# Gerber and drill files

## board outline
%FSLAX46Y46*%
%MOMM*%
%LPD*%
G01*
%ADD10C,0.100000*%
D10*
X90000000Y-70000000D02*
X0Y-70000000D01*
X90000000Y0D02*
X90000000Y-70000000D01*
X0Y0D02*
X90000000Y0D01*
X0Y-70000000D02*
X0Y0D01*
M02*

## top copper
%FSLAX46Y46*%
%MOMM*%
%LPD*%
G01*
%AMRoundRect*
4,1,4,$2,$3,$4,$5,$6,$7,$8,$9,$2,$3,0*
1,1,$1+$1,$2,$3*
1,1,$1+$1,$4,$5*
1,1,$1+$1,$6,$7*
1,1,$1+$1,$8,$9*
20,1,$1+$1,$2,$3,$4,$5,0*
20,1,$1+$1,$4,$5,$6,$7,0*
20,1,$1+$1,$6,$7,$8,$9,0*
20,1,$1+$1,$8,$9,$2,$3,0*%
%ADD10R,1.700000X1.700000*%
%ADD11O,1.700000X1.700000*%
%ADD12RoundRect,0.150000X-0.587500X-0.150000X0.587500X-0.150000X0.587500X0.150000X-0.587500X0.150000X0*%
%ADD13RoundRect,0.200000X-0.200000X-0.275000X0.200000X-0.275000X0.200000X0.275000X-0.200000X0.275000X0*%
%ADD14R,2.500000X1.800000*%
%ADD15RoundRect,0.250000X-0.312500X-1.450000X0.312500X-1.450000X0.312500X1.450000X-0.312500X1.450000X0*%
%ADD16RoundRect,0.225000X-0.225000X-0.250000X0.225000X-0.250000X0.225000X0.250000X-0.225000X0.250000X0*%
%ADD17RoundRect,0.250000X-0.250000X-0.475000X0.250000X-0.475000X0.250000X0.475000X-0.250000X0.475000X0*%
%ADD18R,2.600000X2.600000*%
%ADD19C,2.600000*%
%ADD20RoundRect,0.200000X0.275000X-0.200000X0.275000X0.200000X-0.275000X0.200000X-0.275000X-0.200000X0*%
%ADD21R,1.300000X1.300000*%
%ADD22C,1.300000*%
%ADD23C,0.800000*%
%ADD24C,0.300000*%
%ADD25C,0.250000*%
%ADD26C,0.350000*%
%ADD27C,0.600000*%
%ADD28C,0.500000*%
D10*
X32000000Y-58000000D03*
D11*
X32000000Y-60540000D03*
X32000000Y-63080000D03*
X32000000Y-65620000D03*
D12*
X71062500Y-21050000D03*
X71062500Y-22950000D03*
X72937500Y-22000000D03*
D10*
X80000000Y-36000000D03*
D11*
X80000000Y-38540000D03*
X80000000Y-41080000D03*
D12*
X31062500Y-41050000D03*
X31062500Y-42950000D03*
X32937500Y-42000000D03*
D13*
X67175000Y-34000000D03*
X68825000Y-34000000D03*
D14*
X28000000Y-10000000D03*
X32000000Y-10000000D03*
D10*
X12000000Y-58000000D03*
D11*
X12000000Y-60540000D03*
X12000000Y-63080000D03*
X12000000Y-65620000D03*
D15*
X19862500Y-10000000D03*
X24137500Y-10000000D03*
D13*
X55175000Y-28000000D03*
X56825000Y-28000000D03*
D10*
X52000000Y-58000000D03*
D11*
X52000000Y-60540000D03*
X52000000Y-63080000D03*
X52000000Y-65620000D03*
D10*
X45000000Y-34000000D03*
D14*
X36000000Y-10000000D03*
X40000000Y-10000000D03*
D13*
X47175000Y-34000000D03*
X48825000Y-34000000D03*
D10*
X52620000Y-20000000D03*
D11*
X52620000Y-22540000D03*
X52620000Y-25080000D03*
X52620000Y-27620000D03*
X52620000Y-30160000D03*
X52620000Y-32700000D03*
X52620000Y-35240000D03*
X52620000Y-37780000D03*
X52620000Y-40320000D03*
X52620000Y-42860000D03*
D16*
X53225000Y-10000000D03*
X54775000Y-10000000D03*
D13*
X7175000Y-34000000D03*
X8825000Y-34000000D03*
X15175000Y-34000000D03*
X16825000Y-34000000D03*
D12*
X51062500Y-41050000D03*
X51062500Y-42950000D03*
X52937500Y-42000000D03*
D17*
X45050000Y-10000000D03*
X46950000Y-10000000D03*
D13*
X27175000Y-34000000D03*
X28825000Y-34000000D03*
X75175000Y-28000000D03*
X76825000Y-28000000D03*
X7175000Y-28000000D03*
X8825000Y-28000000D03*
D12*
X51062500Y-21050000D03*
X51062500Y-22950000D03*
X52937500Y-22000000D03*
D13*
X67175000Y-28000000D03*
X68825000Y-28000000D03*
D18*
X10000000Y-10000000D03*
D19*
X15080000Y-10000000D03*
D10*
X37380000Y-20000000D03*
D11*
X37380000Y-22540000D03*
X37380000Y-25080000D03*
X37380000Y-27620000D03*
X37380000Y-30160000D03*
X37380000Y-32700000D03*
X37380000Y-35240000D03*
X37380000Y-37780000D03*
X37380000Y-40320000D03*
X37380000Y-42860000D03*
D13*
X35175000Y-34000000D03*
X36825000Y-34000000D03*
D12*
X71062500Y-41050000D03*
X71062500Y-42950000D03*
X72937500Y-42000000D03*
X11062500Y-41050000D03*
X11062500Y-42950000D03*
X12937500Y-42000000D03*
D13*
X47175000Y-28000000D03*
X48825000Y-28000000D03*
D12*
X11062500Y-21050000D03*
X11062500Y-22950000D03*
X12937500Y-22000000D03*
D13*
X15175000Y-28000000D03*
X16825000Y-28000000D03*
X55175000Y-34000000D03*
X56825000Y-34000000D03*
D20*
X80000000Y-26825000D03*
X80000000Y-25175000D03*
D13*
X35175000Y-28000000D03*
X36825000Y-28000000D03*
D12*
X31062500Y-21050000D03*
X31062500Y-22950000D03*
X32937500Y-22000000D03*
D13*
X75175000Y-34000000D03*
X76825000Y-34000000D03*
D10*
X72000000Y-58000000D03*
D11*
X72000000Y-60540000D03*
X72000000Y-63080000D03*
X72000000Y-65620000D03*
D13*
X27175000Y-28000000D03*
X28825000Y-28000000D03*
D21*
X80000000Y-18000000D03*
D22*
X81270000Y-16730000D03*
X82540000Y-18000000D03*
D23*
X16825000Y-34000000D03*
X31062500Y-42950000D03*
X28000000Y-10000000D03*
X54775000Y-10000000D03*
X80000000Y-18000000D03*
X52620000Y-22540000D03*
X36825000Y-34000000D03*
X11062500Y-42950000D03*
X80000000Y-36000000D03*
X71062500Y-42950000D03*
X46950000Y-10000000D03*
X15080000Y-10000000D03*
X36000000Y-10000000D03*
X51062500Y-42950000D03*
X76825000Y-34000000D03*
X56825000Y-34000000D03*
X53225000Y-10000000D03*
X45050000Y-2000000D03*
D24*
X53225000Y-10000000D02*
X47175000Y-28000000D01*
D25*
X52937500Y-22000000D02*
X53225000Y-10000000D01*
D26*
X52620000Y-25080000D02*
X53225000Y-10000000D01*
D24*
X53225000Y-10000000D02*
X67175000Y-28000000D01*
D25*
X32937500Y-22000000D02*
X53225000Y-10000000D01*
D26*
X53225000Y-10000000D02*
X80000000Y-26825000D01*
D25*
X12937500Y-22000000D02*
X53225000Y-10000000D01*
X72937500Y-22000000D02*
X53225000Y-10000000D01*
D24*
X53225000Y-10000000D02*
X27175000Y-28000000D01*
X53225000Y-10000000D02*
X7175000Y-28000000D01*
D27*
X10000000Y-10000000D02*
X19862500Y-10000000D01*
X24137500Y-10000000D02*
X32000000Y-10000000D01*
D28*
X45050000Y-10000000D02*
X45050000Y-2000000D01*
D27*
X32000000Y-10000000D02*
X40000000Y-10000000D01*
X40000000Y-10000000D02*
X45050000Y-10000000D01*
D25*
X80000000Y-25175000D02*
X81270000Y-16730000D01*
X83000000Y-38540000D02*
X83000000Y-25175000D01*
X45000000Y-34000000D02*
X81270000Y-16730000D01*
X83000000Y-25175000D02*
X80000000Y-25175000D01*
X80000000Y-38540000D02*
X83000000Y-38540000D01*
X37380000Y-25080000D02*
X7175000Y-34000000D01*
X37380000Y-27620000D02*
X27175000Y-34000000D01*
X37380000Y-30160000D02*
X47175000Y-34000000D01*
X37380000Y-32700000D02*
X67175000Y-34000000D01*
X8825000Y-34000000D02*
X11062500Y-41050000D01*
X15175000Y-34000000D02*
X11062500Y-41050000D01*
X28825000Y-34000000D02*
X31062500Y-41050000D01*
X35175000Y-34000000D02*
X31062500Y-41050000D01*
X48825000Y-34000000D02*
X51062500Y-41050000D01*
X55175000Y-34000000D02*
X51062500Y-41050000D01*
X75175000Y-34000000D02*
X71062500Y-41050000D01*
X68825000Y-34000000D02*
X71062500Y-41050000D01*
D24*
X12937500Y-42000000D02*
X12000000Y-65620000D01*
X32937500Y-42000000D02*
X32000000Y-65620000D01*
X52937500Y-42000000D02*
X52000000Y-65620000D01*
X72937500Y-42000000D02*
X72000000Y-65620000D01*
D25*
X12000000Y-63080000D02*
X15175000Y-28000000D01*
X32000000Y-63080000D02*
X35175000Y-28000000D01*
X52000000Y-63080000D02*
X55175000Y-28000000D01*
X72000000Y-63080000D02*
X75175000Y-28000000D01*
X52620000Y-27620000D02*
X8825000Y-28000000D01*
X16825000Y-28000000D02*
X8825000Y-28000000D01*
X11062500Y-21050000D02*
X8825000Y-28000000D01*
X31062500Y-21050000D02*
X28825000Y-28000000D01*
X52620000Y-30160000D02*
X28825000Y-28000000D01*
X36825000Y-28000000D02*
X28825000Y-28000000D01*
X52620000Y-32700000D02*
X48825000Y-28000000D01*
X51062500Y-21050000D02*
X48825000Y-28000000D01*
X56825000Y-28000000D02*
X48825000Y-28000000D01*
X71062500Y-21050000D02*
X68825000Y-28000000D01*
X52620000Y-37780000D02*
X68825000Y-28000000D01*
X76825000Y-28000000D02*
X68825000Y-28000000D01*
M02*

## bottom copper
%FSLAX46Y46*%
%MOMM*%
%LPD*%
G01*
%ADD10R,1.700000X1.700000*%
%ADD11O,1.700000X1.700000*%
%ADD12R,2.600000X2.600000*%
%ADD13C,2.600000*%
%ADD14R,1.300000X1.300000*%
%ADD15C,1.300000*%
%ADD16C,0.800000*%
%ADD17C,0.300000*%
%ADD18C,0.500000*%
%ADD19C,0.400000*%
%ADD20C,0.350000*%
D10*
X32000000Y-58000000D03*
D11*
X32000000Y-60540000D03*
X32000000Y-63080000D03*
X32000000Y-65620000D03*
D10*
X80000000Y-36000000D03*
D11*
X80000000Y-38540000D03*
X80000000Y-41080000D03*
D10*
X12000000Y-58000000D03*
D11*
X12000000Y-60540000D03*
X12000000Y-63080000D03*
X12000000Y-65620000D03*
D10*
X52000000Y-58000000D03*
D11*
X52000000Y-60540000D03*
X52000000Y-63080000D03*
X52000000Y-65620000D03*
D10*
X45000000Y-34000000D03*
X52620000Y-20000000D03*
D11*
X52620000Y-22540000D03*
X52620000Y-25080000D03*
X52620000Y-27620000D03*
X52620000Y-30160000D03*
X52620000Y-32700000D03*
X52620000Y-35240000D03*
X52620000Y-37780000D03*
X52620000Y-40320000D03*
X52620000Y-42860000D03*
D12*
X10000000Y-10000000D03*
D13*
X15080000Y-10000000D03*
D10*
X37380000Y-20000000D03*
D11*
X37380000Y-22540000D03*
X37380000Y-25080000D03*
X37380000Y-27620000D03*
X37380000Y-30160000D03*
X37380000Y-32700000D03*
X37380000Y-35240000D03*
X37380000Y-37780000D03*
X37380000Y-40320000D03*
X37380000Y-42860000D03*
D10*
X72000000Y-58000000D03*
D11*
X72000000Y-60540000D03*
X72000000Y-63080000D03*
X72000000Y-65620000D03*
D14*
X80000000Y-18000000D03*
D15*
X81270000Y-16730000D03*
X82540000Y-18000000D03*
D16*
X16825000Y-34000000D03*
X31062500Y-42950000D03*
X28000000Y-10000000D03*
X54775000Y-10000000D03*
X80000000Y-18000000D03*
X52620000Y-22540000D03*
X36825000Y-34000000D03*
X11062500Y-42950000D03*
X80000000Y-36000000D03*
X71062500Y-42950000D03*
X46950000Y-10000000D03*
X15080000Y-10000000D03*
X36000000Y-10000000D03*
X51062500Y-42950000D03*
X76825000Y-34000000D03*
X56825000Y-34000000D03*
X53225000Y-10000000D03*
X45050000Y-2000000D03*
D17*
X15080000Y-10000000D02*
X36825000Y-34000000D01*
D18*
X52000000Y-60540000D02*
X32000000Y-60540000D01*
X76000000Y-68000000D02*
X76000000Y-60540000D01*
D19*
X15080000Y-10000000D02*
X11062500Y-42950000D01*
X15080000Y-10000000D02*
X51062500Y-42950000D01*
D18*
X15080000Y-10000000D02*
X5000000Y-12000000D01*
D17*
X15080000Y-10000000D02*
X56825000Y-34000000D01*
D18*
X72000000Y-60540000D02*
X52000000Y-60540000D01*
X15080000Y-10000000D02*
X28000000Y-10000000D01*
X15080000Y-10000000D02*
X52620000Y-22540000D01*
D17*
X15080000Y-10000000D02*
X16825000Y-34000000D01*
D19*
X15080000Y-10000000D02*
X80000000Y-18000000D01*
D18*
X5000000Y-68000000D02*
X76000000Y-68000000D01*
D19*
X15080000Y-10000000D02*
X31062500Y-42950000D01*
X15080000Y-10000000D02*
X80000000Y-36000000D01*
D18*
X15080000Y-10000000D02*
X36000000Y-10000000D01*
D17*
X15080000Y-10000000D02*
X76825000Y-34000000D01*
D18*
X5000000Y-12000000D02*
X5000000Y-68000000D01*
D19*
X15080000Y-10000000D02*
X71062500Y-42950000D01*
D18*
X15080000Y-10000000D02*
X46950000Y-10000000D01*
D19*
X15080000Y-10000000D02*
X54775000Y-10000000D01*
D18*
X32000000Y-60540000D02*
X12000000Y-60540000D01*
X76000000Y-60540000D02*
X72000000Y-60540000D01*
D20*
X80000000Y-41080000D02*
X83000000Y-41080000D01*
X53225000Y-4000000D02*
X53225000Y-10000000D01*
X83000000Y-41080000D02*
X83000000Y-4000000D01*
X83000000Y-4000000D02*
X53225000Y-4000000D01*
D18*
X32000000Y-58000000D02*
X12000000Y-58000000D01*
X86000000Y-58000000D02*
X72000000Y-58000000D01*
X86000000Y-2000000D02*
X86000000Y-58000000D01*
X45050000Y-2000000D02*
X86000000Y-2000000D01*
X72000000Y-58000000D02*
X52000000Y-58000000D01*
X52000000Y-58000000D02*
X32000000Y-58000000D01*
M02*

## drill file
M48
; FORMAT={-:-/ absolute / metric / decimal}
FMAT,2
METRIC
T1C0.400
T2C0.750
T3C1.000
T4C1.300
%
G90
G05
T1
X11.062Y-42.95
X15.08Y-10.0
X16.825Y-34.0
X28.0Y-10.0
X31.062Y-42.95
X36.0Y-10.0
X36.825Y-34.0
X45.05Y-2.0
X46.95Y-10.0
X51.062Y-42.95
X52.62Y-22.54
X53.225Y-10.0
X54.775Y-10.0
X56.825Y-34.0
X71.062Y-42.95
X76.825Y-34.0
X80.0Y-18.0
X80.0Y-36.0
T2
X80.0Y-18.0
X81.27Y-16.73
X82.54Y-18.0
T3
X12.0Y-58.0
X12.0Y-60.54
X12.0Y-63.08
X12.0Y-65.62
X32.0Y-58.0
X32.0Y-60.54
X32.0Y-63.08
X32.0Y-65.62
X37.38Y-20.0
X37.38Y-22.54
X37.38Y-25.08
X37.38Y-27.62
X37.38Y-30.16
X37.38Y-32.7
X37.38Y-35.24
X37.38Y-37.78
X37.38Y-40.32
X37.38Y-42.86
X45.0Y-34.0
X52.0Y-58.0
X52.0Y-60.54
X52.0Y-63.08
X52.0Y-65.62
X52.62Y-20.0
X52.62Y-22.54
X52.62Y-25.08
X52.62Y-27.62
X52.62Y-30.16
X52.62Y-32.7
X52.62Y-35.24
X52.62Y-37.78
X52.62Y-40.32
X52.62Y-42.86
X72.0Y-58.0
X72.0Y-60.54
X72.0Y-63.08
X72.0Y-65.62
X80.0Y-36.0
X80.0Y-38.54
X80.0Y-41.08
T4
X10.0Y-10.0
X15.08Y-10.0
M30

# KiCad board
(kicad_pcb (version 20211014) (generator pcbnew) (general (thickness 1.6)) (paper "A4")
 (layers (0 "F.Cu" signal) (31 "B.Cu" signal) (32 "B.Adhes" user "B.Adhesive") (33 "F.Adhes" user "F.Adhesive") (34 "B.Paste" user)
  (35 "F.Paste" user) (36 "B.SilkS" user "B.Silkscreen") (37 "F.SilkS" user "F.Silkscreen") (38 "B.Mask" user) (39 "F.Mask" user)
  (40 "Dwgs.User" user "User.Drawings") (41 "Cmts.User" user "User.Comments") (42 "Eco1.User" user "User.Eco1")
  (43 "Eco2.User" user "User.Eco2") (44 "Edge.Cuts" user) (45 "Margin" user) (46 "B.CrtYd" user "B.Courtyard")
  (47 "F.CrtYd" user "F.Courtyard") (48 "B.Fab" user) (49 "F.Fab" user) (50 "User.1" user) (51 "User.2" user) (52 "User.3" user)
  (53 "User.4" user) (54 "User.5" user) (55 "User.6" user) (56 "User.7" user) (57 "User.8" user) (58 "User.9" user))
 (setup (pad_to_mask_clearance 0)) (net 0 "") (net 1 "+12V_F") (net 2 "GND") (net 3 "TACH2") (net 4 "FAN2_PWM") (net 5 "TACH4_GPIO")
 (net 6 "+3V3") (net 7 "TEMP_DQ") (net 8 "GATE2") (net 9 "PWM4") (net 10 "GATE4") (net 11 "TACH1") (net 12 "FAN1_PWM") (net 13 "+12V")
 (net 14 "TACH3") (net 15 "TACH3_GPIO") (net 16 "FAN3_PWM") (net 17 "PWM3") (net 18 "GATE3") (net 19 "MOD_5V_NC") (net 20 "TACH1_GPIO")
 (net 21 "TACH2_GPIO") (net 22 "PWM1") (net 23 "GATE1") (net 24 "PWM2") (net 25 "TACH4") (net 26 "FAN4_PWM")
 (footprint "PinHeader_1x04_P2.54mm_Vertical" (layer "F.Cu") (at 32 58)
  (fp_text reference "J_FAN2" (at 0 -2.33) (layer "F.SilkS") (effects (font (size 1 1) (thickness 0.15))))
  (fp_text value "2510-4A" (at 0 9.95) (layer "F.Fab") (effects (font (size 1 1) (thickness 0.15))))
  (pad "1" thru_hole rect (at 0 0) (size 1.7 1.7) (drill 1) (layers *.Cu *.Mask) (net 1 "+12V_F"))
  (pad "2" thru_hole oval (at 0 2.54) (size 1.7 1.7) (drill 1) (layers *.Cu *.Mask) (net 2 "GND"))
  (pad "3" thru_hole oval (at 0 5.08) (size 1.7 1.7) (drill 1) (layers *.Cu *.Mask) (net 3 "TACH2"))
  (pad "4" thru_hole oval (at 0 7.62) (size 1.7 1.7) (drill 1) (layers *.Cu *.Mask) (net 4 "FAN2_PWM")))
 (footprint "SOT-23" (layer "F.Cu") (at 72 22)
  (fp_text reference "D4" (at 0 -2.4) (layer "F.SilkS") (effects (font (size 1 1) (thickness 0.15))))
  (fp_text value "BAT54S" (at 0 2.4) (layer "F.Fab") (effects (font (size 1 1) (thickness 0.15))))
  (pad "1" smd roundrect (at -0.9375 -0.95) (size 1.475 0.6) (layers "F.Cu" "F.Paste" "F.Mask") (roundrect_rratio 0.25) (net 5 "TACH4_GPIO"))
  (pad "2" smd roundrect (at -0.9375 0.95) (size 1.475 0.6) (layers "F.Cu" "F.Paste" "F.Mask") (roundrect_rratio 0.25) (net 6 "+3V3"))
  (pad "3" smd roundrect (at 0.9375 0) (size 1.475 0.6) (layers "F.Cu" "F.Paste" "F.Mask") (roundrect_rratio 0.25) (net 6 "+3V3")))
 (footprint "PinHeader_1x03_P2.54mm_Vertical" (layer "F.Cu") (at 80 36)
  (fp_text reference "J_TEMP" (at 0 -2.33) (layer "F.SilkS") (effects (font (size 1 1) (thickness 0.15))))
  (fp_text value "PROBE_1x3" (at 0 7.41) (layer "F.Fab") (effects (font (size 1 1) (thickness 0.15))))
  (pad "1" thru_hole rect (at 0 0) (size 1.7 1.7) (drill 1) (layers *.Cu *.Mask) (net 2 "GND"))
  (pad "2" thru_hole oval (at 0 2.54) (size 1.7 1.7) (drill 1) (layers *.Cu *.Mask) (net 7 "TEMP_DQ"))
  (pad "3" thru_hole oval (at 0 5.08) (size 1.7 1.7) (drill 1) (layers *.Cu *.Mask) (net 6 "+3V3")))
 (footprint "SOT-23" (layer "F.Cu") (at 32 42)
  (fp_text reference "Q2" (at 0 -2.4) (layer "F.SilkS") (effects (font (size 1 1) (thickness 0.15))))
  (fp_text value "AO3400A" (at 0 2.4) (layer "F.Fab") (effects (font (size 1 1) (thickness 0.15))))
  (pad "1" smd roundrect (at -0.9375 -0.95) (size 1.475 0.6) (layers "F.Cu" "F.Paste" "F.Mask") (roundrect_rratio 0.25) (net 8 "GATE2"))
  (pad "2" smd roundrect (at -0.9375 0.95) (size 1.475 0.6) (layers "F.Cu" "F.Paste" "F.Mask") (roundrect_rratio 0.25) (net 2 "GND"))
  (pad "3" smd roundrect (at 0.9375 0) (size 1.475 0.6) (layers "F.Cu" "F.Paste" "F.Mask") (roundrect_rratio 0.25) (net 4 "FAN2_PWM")))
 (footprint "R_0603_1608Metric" (layer "F.Cu") (at 68 34)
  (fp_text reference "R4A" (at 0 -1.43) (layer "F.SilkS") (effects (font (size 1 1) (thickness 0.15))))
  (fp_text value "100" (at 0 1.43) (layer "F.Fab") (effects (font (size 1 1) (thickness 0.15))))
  (pad "1" smd roundrect (at -0.825 0) (size 0.8 0.95) (layers "F.Cu" "F.Paste" "F.Mask") (roundrect_rratio 0.25) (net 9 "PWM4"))
  (pad "2" smd roundrect (at 0.825 0) (size 0.8 0.95) (layers "F.Cu" "F.Paste" "F.Mask") (roundrect_rratio 0.25) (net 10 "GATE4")))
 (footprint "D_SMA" (layer "F.Cu") (at 30 10)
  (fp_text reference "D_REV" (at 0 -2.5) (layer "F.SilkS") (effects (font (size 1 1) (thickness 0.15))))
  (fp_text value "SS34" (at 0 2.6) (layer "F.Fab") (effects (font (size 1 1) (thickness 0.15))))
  (pad "1" smd rect (at -2 0) (size 2.5 1.8) (layers "F.Cu" "F.Paste" "F.Mask") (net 2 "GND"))
  (pad "2" smd rect (at 2 0) (size 2.5 1.8) (layers "F.Cu" "F.Paste" "F.Mask") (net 1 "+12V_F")))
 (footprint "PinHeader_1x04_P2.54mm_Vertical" (layer "F.Cu") (at 12 58)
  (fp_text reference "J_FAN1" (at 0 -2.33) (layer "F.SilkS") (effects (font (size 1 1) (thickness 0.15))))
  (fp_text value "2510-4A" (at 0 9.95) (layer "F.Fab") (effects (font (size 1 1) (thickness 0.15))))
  (pad "1" thru_hole rect (at 0 0) (size 1.7 1.7) (drill 1) (layers *.Cu *.Mask) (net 1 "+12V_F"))
  (pad "2" thru_hole oval (at 0 2.54) (size 1.7 1.7) (drill 1) (layers *.Cu *.Mask) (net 2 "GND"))
  (pad "3" thru_hole oval (at 0 5.08) (size 1.7 1.7) (drill 1) (layers *.Cu *.Mask) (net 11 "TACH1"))
  (pad "4" thru_hole oval (at 0 7.62) (size 1.7 1.7) (drill 1) (layers *.Cu *.Mask) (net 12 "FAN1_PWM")))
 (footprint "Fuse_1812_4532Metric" (layer "F.Cu") (at 22 10)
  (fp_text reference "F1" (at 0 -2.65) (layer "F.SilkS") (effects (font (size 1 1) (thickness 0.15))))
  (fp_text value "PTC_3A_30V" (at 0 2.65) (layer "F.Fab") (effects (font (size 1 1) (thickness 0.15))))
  (pad "1" smd roundrect (at -2.1375 0) (size 1.125 3.4) (layers "F.Cu" "F.Paste" "F.Mask") (roundrect_rratio 0.222222) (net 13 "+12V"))
  (pad "2" smd roundrect (at 2.1375 0) (size 1.125 3.4) (layers "F.Cu" "F.Paste" "F.Mask") (roundrect_rratio 0.222222) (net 1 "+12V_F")))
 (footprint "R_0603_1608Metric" (layer "F.Cu") (at 56 28)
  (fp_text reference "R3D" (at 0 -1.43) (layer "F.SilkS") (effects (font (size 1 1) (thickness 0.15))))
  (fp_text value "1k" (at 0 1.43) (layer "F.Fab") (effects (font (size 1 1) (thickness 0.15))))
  (pad "1" smd roundrect (at -0.825 0) (size 0.8 0.95) (layers "F.Cu" "F.Paste" "F.Mask") (roundrect_rratio 0.25) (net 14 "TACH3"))
  (pad "2" smd roundrect (at 0.825 0) (size 0.8 0.95) (layers "F.Cu" "F.Paste" "F.Mask") (roundrect_rratio 0.25) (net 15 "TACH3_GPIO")))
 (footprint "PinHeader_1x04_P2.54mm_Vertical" (layer "F.Cu") (at 52 58)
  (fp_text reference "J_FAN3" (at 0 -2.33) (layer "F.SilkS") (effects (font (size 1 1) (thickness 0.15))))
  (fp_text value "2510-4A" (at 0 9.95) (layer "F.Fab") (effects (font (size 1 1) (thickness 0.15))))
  (pad "1" thru_hole rect (at 0 0) (size 1.7 1.7) (drill 1) (layers *.Cu *.Mask) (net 1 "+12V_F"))
  (pad "2" thru_hole oval (at 0 2.54) (size 1.7 1.7) (drill 1) (layers *.Cu *.Mask) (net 2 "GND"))
  (pad "3" thru_hole oval (at 0 5.08) (size 1.7 1.7) (drill 1) (layers *.Cu *.Mask) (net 14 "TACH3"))
  (pad "4" thru_hole oval (at 0 7.62) (size 1.7 1.7) (drill 1) (layers *.Cu *.Mask) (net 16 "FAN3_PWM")))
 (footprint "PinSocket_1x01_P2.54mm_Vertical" (layer "F.Cu") (at 45 34)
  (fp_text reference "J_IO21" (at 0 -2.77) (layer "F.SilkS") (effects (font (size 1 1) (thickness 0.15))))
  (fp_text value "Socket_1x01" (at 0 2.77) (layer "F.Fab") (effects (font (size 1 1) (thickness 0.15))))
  (pad "1" thru_hole rect (at 0 0) (size 1.7 1.7) (drill 1) (layers *.Cu *.Mask) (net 7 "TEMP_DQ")))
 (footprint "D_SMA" (layer "F.Cu") (at 38 10)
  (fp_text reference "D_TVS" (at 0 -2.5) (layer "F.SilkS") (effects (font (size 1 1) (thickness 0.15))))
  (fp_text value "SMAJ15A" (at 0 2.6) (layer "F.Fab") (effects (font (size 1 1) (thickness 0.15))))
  (pad "1" smd rect (at -2 0) (size 2.5 1.8) (layers "F.Cu" "F.Paste" "F.Mask") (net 2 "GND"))
  (pad "2" smd rect (at 2 0) (size 2.5 1.8) (layers "F.Cu" "F.Paste" "F.Mask") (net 1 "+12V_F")))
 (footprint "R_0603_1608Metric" (layer "F.Cu") (at 48 34)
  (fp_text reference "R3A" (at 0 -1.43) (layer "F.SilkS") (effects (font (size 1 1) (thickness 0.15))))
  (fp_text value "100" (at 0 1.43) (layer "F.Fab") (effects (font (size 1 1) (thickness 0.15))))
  (pad "1" smd roundrect (at -0.825 0) (size 0.8 0.95) (layers "F.Cu" "F.Paste" "F.Mask") (roundrect_rratio 0.25) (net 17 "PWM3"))
  (pad "2" smd roundrect (at 0.825 0) (size 0.8 0.95) (layers "F.Cu" "F.Paste" "F.Mask") (roundrect_rratio 0.25) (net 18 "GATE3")))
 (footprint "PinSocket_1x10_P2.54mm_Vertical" (layer "F.Cu") (at 52.62 20)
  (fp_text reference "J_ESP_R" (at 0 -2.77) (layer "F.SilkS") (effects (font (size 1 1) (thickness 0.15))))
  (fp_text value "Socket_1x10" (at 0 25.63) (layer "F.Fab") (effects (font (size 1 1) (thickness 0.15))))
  (pad "1" thru_hole rect (at 0 0) (size 1.7 1.7) (drill 1) (layers *.Cu *.Mask) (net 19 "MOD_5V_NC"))
  (pad "2" thru_hole oval (at 0 2.54) (size 1.7 1.7) (drill 1) (layers *.Cu *.Mask) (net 2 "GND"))
  (pad "3" thru_hole oval (at 0 5.08) (size 1.7 1.7) (drill 1) (layers *.Cu *.Mask) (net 6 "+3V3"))
  (pad "4" thru_hole oval (at 0 7.62) (size 1.7 1.7) (drill 1) (layers *.Cu *.Mask) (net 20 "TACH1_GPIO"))
  (pad "5" thru_hole oval (at 0 10.16) (size 1.7 1.7) (drill 1) (layers *.Cu *.Mask) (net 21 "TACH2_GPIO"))
  (pad "6" thru_hole oval (at 0 12.7) (size 1.7 1.7) (drill 1) (layers *.Cu *.Mask) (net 15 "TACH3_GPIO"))
  (pad "7" thru_hole oval (at 0 15.24) (size 1.7 1.7) (drill 1) (layers *.Cu *.Mask))
  (pad "8" thru_hole oval (at 0 17.78) (size 1.7 1.7) (drill 1) (layers *.Cu *.Mask) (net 5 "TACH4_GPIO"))
  (pad "9" thru_hole oval (at 0 20.32) (size 1.7 1.7) (drill 1) (layers *.Cu *.Mask))
  (pad "10" thru_hole oval (at 0 22.86) (size 1.7 1.7) (drill 1) (layers *.Cu *.Mask)))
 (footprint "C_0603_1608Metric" (layer "F.Cu") (at 54 10)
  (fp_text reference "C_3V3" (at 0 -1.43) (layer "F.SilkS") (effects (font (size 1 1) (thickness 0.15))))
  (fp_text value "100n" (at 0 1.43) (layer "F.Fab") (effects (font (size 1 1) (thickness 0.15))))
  (pad "1" smd roundrect (at -0.775 0) (size 0.9 0.95) (layers "F.Cu" "F.Paste" "F.Mask") (roundrect_rratio 0.25) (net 6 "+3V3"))
  (pad "2" smd roundrect (at 0.775 0) (size 0.9 0.95) (layers "F.Cu" "F.Paste" "F.Mask") (roundrect_rratio 0.25) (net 2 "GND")))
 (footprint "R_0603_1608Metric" (layer "F.Cu") (at 8 34)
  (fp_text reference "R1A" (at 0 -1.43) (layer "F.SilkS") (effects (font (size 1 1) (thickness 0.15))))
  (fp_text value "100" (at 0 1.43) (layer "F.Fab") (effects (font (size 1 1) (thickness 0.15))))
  (pad "1" smd roundrect (at -0.825 0) (size 0.8 0.95) (layers "F.Cu" "F.Paste" "F.Mask") (roundrect_rratio 0.25) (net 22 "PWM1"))
  (pad "2" smd roundrect (at 0.825 0) (size 0.8 0.95) (layers "F.Cu" "F.Paste" "F.Mask") (roundrect_rratio 0.25) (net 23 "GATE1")))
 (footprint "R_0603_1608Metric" (layer "F.Cu") (at 16 34)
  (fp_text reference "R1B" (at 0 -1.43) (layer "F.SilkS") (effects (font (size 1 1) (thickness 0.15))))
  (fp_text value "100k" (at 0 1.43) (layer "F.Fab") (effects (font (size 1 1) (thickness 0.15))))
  (pad "1" smd roundrect (at -0.825 0) (size 0.8 0.95) (layers "F.Cu" "F.Paste" "F.Mask") (roundrect_rratio 0.25) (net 23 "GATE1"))
  (pad "2" smd roundrect (at 0.825 0) (size 0.8 0.95) (layers "F.Cu" "F.Paste" "F.Mask") (roundrect_rratio 0.25) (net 2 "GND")))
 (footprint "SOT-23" (layer "F.Cu") (at 52 42)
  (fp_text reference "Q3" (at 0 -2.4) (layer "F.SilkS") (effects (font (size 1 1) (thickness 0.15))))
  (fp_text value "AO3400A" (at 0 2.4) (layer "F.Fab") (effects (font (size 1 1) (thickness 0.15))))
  (pad "1" smd roundrect (at -0.9375 -0.95) (size 1.475 0.6) (layers "F.Cu" "F.Paste" "F.Mask") (roundrect_rratio 0.25) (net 18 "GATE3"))
  (pad "2" smd roundrect (at -0.9375 0.95) (size 1.475 0.6) (layers "F.Cu" "F.Paste" "F.Mask") (roundrect_rratio 0.25) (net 2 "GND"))
  (pad "3" smd roundrect (at 0.9375 0) (size 1.475 0.6) (layers "F.Cu" "F.Paste" "F.Mask") (roundrect_rratio 0.25) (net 16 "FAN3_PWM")))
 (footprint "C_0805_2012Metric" (layer "F.Cu") (at 46 10)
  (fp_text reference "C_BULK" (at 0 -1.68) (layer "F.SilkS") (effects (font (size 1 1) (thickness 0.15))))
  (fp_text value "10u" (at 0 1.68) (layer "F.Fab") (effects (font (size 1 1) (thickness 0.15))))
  (pad "1" smd roundrect (at -0.95 0) (size 1 1.45) (layers "F.Cu" "F.Paste" "F.Mask") (roundrect_rratio 0.25) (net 1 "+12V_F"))
  (pad "2" smd roundrect (at 0.95 0) (size 1 1.45) (layers "F.Cu" "F.Paste" "F.Mask") (roundrect_rratio 0.25) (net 2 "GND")))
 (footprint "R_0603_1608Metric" (layer "F.Cu") (at 28 34)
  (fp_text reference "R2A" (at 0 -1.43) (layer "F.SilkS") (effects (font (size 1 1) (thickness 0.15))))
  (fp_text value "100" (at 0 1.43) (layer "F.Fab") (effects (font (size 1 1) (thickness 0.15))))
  (pad "1" smd roundrect (at -0.825 0) (size 0.8 0.95) (layers "F.Cu" "F.Paste" "F.Mask") (roundrect_rratio 0.25) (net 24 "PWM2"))
  (pad "2" smd roundrect (at 0.825 0) (size 0.8 0.95) (layers "F.Cu" "F.Paste" "F.Mask") (roundrect_rratio 0.25) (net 8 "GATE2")))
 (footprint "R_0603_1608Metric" (layer "F.Cu") (at 76 28)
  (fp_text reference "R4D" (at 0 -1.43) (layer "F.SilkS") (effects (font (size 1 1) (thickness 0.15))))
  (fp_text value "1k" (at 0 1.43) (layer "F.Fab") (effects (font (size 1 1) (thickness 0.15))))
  (pad "1" smd roundrect (at -0.825 0) (size 0.8 0.95) (layers "F.Cu" "F.Paste" "F.Mask") (roundrect_rratio 0.25) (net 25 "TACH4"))
  (pad "2" smd roundrect (at 0.825 0) (size 0.8 0.95) (layers "F.Cu" "F.Paste" "F.Mask") (roundrect_rratio 0.25) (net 5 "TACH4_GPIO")))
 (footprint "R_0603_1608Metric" (layer "F.Cu") (at 8 28)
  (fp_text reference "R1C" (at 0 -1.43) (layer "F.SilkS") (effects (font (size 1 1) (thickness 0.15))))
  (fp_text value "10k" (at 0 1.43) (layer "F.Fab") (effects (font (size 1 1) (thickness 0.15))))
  (pad "1" smd roundrect (at -0.825 0) (size 0.8 0.95) (layers "F.Cu" "F.Paste" "F.Mask") (roundrect_rratio 0.25) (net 6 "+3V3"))
  (pad "2" smd roundrect (at 0.825 0) (size 0.8 0.95) (layers "F.Cu" "F.Paste" "F.Mask") (roundrect_rratio 0.25) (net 20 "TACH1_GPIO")))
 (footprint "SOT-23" (layer "F.Cu") (at 52 22)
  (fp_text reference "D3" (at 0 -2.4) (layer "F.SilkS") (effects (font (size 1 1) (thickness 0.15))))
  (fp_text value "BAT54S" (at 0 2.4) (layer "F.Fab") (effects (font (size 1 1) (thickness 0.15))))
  (pad "1" smd roundrect (at -0.9375 -0.95) (size 1.475 0.6) (layers "F.Cu" "F.Paste" "F.Mask") (roundrect_rratio 0.25)
   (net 15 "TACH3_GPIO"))
  (pad "2" smd roundrect (at -0.9375 0.95) (size 1.475 0.6) (layers "F.Cu" "F.Paste" "F.Mask") (roundrect_rratio 0.25) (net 6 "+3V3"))
  (pad "3" smd roundrect (at 0.9375 0) (size 1.475 0.6) (layers "F.Cu" "F.Paste" "F.Mask") (roundrect_rratio 0.25) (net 6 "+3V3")))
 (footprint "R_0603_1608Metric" (layer "F.Cu") (at 68 28)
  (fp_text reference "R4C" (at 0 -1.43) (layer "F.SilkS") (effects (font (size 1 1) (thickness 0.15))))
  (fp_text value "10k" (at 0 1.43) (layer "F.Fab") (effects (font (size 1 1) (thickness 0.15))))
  (pad "1" smd roundrect (at -0.825 0) (size 0.8 0.95) (layers "F.Cu" "F.Paste" "F.Mask") (roundrect_rratio 0.25) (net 6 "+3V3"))
  (pad "2" smd roundrect (at 0.825 0) (size 0.8 0.95) (layers "F.Cu" "F.Paste" "F.Mask") (roundrect_rratio 0.25) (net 5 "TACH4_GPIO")))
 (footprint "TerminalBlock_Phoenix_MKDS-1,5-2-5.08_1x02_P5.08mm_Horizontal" (layer "F.Cu") (at 10 10)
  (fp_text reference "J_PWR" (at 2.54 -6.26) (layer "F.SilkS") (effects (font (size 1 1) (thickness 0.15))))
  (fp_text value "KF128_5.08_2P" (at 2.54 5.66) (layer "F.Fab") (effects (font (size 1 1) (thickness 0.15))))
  (pad "1" thru_hole rect (at 0 0) (size 2.6 2.6) (drill 1.3) (layers *.Cu *.Mask) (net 13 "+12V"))
  (pad "2" thru_hole circle (at 5.08 0) (size 2.6 2.6) (drill 1.3) (layers *.Cu *.Mask) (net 2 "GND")))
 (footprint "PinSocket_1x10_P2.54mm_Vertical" (layer "F.Cu") (at 37.38 20)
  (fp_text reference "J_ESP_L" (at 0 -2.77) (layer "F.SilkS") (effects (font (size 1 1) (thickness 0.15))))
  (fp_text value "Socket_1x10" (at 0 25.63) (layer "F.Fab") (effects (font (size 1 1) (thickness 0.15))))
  (pad "1" thru_hole rect (at 0 0) (size 1.7 1.7) (drill 1) (layers *.Cu *.Mask))
  (pad "2" thru_hole oval (at 0 2.54) (size 1.7 1.7) (drill 1) (layers *.Cu *.Mask))
  (pad "3" thru_hole oval (at 0 5.08) (size 1.7 1.7) (drill 1) (layers *.Cu *.Mask) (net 22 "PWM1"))
  (pad "4" thru_hole oval (at 0 7.62) (size 1.7 1.7) (drill 1) (layers *.Cu *.Mask) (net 24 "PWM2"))
  (pad "5" thru_hole oval (at 0 10.16) (size 1.7 1.7) (drill 1) (layers *.Cu *.Mask) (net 17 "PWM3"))
  (pad "6" thru_hole oval (at 0 12.7) (size 1.7 1.7) (drill 1) (layers *.Cu *.Mask) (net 9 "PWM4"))
  (pad "7" thru_hole oval (at 0 15.24) (size 1.7 1.7) (drill 1) (layers *.Cu *.Mask))
  (pad "8" thru_hole oval (at 0 17.78) (size 1.7 1.7) (drill 1) (layers *.Cu *.Mask))
  (pad "9" thru_hole oval (at 0 20.32) (size 1.7 1.7) (drill 1) (layers *.Cu *.Mask))
  (pad "10" thru_hole oval (at 0 22.86) (size 1.7 1.7) (drill 1) (layers *.Cu *.Mask)))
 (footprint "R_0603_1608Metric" (layer "F.Cu") (at 36 34)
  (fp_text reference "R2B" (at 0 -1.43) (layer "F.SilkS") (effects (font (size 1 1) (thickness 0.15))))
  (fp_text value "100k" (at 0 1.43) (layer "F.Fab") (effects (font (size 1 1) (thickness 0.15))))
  (pad "1" smd roundrect (at -0.825 0) (size 0.8 0.95) (layers "F.Cu" "F.Paste" "F.Mask") (roundrect_rratio 0.25) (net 8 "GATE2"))
  (pad "2" smd roundrect (at 0.825 0) (size 0.8 0.95) (layers "F.Cu" "F.Paste" "F.Mask") (roundrect_rratio 0.25) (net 2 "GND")))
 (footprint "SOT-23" (layer "F.Cu") (at 72 42)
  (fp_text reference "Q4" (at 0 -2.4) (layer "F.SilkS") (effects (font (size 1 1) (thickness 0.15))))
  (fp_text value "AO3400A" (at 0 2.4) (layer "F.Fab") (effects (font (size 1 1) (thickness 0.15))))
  (pad "1" smd roundrect (at -0.9375 -0.95) (size 1.475 0.6) (layers "F.Cu" "F.Paste" "F.Mask") (roundrect_rratio 0.25) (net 10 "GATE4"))
  (pad "2" smd roundrect (at -0.9375 0.95) (size 1.475 0.6) (layers "F.Cu" "F.Paste" "F.Mask") (roundrect_rratio 0.25) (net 2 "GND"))
  (pad "3" smd roundrect (at 0.9375 0) (size 1.475 0.6) (layers "F.Cu" "F.Paste" "F.Mask") (roundrect_rratio 0.25) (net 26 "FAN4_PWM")))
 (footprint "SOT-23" (layer "F.Cu") (at 12 42)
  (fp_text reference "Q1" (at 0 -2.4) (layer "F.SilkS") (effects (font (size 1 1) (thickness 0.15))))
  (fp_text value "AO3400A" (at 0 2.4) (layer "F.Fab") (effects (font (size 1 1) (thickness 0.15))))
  (pad "1" smd roundrect (at -0.9375 -0.95) (size 1.475 0.6) (layers "F.Cu" "F.Paste" "F.Mask") (roundrect_rratio 0.25) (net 23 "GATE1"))
  (pad "2" smd roundrect (at -0.9375 0.95) (size 1.475 0.6) (layers "F.Cu" "F.Paste" "F.Mask") (roundrect_rratio 0.25) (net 2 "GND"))
  (pad "3" smd roundrect (at 0.9375 0) (size 1.475 0.6) (layers "F.Cu" "F.Paste" "F.Mask") (roundrect_rratio 0.25) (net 12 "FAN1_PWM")))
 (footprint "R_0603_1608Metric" (layer "F.Cu") (at 48 28)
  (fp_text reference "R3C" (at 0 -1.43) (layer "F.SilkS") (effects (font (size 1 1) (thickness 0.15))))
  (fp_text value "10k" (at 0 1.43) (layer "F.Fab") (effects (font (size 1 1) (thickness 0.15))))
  (pad "1" smd roundrect (at -0.825 0) (size 0.8 0.95) (layers "F.Cu" "F.Paste" "F.Mask") (roundrect_rratio 0.25) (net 6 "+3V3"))
  (pad "2" smd roundrect (at 0.825 0) (size 0.8 0.95) (layers "F.Cu" "F.Paste" "F.Mask") (roundrect_rratio 0.25) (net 15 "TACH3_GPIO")))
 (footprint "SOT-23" (layer "F.Cu") (at 12 22)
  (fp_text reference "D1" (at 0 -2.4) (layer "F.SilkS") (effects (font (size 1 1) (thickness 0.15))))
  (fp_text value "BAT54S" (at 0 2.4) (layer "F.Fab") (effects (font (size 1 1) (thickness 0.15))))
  (pad "1" smd roundrect (at -0.9375 -0.95) (size 1.475 0.6) (layers "F.Cu" "F.Paste" "F.Mask") (roundrect_rratio 0.25)
   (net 20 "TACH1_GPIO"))
  (pad "2" smd roundrect (at -0.9375 0.95) (size 1.475 0.6) (layers "F.Cu" "F.Paste" "F.Mask") (roundrect_rratio 0.25) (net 6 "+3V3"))
  (pad "3" smd roundrect (at 0.9375 0) (size 1.475 0.6) (layers "F.Cu" "F.Paste" "F.Mask") (roundrect_rratio 0.25) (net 6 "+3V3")))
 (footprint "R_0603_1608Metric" (layer "F.Cu") (at 16 28)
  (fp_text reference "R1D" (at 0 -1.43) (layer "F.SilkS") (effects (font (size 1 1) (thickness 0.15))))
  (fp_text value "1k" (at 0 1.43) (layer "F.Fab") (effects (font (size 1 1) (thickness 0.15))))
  (pad "1" smd roundrect (at -0.825 0) (size 0.8 0.95) (layers "F.Cu" "F.Paste" "F.Mask") (roundrect_rratio 0.25) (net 11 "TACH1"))
  (pad "2" smd roundrect (at 0.825 0) (size 0.8 0.95) (layers "F.Cu" "F.Paste" "F.Mask") (roundrect_rratio 0.25) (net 20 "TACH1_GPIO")))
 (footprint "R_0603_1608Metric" (layer "F.Cu") (at 56 34)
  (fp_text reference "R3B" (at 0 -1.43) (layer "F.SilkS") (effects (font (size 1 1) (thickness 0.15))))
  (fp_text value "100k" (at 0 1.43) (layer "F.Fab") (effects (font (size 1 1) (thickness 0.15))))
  (pad "1" smd roundrect (at -0.825 0) (size 0.8 0.95) (layers "F.Cu" "F.Paste" "F.Mask") (roundrect_rratio 0.25) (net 18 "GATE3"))
  (pad "2" smd roundrect (at 0.825 0) (size 0.8 0.95) (layers "F.Cu" "F.Paste" "F.Mask") (roundrect_rratio 0.25) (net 2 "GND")))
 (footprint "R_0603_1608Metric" (layer "F.Cu") (at 80 26 90)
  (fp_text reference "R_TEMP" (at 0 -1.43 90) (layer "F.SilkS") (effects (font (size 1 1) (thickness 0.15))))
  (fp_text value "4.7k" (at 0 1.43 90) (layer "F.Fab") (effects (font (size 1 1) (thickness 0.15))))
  (pad "1" smd roundrect (at -0.825 0 90) (size 0.8 0.95) (layers "F.Cu" "F.Paste" "F.Mask") (roundrect_rratio 0.25) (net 6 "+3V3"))
  (pad "2" smd roundrect (at 0.825 0 90) (size 0.8 0.95) (layers "F.Cu" "F.Paste" "F.Mask") (roundrect_rratio 0.25) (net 7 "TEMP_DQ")))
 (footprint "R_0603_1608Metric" (layer "F.Cu") (at 36 28)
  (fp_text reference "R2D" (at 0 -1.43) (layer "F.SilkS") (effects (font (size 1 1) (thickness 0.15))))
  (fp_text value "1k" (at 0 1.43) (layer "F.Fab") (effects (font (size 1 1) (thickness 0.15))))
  (pad "1" smd roundrect (at -0.825 0) (size 0.8 0.95) (layers "F.Cu" "F.Paste" "F.Mask") (roundrect_rratio 0.25) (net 3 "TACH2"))
  (pad "2" smd roundrect (at 0.825 0) (size 0.8 0.95) (layers "F.Cu" "F.Paste" "F.Mask") (roundrect_rratio 0.25) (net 21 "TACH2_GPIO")))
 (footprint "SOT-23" (layer "F.Cu") (at 32 22)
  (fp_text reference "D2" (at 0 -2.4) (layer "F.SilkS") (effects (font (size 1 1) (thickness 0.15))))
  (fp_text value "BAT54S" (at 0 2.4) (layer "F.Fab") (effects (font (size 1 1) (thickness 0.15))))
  (pad "1" smd roundrect (at -0.9375 -0.95) (size 1.475 0.6) (layers "F.Cu" "F.Paste" "F.Mask") (roundrect_rratio 0.25)
   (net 21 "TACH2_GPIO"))
  (pad "2" smd roundrect (at -0.9375 0.95) (size 1.475 0.6) (layers "F.Cu" "F.Paste" "F.Mask") (roundrect_rratio 0.25) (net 6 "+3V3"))
  (pad "3" smd roundrect (at 0.9375 0) (size 1.475 0.6) (layers "F.Cu" "F.Paste" "F.Mask") (roundrect_rratio 0.25) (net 6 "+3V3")))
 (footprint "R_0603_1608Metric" (layer "F.Cu") (at 76 34)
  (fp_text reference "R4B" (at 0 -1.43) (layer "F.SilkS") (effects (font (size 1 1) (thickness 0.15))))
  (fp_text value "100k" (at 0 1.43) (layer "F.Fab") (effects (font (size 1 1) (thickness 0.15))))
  (pad "1" smd roundrect (at -0.825 0) (size 0.8 0.95) (layers "F.Cu" "F.Paste" "F.Mask") (roundrect_rratio 0.25) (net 10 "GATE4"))
  (pad "2" smd roundrect (at 0.825 0) (size 0.8 0.95) (layers "F.Cu" "F.Paste" "F.Mask") (roundrect_rratio 0.25) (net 2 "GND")))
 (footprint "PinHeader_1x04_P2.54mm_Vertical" (layer "F.Cu") (at 72 58)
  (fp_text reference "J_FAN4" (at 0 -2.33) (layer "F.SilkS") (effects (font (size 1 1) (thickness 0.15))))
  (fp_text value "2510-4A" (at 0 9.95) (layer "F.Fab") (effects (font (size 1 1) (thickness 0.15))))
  (pad "1" thru_hole rect (at 0 0) (size 1.7 1.7) (drill 1) (layers *.Cu *.Mask) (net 1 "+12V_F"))
  (pad "2" thru_hole oval (at 0 2.54) (size 1.7 1.7) (drill 1) (layers *.Cu *.Mask) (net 2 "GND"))
  (pad "3" thru_hole oval (at 0 5.08) (size 1.7 1.7) (drill 1) (layers *.Cu *.Mask) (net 25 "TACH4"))
  (pad "4" thru_hole oval (at 0 7.62) (size 1.7 1.7) (drill 1) (layers *.Cu *.Mask) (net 26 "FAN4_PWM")))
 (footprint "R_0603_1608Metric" (layer "F.Cu") (at 28 28)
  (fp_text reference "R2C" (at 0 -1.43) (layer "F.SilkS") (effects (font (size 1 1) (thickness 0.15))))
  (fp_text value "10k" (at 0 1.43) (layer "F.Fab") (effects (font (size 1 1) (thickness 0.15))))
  (pad "1" smd roundrect (at -0.825 0) (size 0.8 0.95) (layers "F.Cu" "F.Paste" "F.Mask") (roundrect_rratio 0.25) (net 6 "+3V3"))
  (pad "2" smd roundrect (at 0.825 0) (size 0.8 0.95) (layers "F.Cu" "F.Paste" "F.Mask") (roundrect_rratio 0.25) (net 21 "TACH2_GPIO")))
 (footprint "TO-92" (layer "F.Cu") (at 80 18)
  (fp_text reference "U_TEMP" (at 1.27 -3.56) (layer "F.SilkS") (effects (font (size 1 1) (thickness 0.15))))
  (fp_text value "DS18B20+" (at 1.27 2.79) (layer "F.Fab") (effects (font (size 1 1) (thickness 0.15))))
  (pad "1" thru_hole rect (at 0 0) (size 1.3 1.3) (drill 0.75) (layers *.Cu *.Mask) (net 2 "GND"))
  (pad "2" thru_hole circle (at 1.27 -1.27) (size 1.3 1.3) (drill 0.75) (layers *.Cu *.Mask) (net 7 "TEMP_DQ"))
  (pad "3" thru_hole circle (at 2.54 0) (size 1.3 1.3) (drill 0.75) (layers *.Cu *.Mask) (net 6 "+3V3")))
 (gr_line (start 90 70) (end 0 70) (layer "Edge.Cuts") (width 0.1))
 (gr_line (start 90 0) (end 90 70) (layer "Edge.Cuts") (width 0.1))
 (gr_line (start 0 0) (end 90 0) (layer "Edge.Cuts") (width 0.1))
 (gr_line (start 0 70) (end 0 0) (layer "Edge.Cuts") (width 0.1))
 (via (at 16.825 34) (size 0.8) (drill 0.4) (layers "F.Cu" "B.Cu") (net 2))
 (via (at 31.0625 42.95) (size 0.8) (drill 0.4) (layers "F.Cu" "B.Cu") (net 2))
 (via (at 28 10) (size 0.8) (drill 0.4) (layers "F.Cu" "B.Cu") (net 2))
 (via (at 54.775 10) (size 0.8) (drill 0.4) (layers "F.Cu" "B.Cu") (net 2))
 (via (at 80 18) (size 0.8) (drill 0.4) (layers "F.Cu" "B.Cu") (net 2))
 (via (at 52.62 22.54) (size 0.8) (drill 0.4) (layers "F.Cu" "B.Cu") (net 2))
 (via (at 36.825 34) (size 0.8) (drill 0.4) (layers "F.Cu" "B.Cu") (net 2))
 (via (at 11.0625 42.95) (size 0.8) (drill 0.4) (layers "F.Cu" "B.Cu") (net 2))
 (via (at 80 36) (size 0.8) (drill 0.4) (layers "F.Cu" "B.Cu") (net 2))
 (via (at 71.0625 42.95) (size 0.8) (drill 0.4) (layers "F.Cu" "B.Cu") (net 2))
 (via (at 46.95 10) (size 0.8) (drill 0.4) (layers "F.Cu" "B.Cu") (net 2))
 (via (at 15.08 10) (size 0.8) (drill 0.4) (layers "F.Cu" "B.Cu") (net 2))
 (via (at 36 10) (size 0.8) (drill 0.4) (layers "F.Cu" "B.Cu") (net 2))
 (via (at 51.0625 42.95) (size 0.8) (drill 0.4) (layers "F.Cu" "B.Cu") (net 2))
 (via (at 76.825 34) (size 0.8) (drill 0.4) (layers "F.Cu" "B.Cu") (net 2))
 (via (at 56.825 34) (size 0.8) (drill 0.4) (layers "F.Cu" "B.Cu") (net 2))
 (segment (start 15.08 10) (end 36.825 34) (width 0.3) (layer "B.Cu") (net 2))
 (segment (start 52 60.54) (end 32 60.54) (width 0.5) (layer "B.Cu") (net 2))
 (segment (start 76 68) (end 76 60.54) (width 0.5) (layer "B.Cu") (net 2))
 (segment (start 15.08 10) (end 11.0625 42.95) (width 0.4) (layer "B.Cu") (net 2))
 (segment (start 15.08 10) (end 51.0625 42.95) (width 0.4) (layer "B.Cu") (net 2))
 (segment (start 15.08 10) (end 5 12) (width 0.5) (layer "B.Cu") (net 2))
 (segment (start 15.08 10) (end 56.825 34) (width 0.3) (layer "B.Cu") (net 2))
 (segment (start 72 60.54) (end 52 60.54) (width 0.5) (layer "B.Cu") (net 2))
 (segment (start 15.08 10) (end 28 10) (width 0.5) (layer "B.Cu") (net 2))
 (segment (start 15.08 10) (end 52.62 22.54) (width 0.5) (layer "B.Cu") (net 2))
 (segment (start 15.08 10) (end 16.825 34) (width 0.3) (layer "B.Cu") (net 2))
 (segment (start 15.08 10) (end 80 18) (width 0.4) (layer "B.Cu") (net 2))
 (segment (start 5 68) (end 76 68) (width 0.5) (layer "B.Cu") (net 2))
 (segment (start 15.08 10) (end 31.0625 42.95) (width 0.4) (layer "B.Cu") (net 2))
 (segment (start 15.08 10) (end 80 36) (width 0.4) (layer "B.Cu") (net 2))
 (segment (start 15.08 10) (end 36 10) (width 0.5) (layer "B.Cu") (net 2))
 (segment (start 15.08 10) (end 76.825 34) (width 0.3) (layer "B.Cu") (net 2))
 (segment (start 5 12) (end 5 68) (width 0.5) (layer "B.Cu") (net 2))
 (segment (start 15.08 10) (end 71.0625 42.95) (width 0.4) (layer "B.Cu") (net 2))
 (segment (start 15.08 10) (end 46.95 10) (width 0.5) (layer "B.Cu") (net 2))
 (segment (start 15.08 10) (end 54.775 10) (width 0.4) (layer "B.Cu") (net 2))
 (segment (start 32 60.54) (end 12 60.54) (width 0.5) (layer "B.Cu") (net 2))
 (segment (start 76 60.54) (end 72 60.54) (width 0.5) (layer "B.Cu") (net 2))
 (segment (start 53.225 10) (end 47.175 28) (width 0.3) (layer "F.Cu") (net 6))
 (segment (start 52.9375 22) (end 53.225 10) (width 0.25) (layer "F.Cu") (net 6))
 (segment (start 52.62 25.08) (end 53.225 10) (width 0.35) (layer "F.Cu") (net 6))
 (segment (start 53.225 10) (end 67.175 28) (width 0.3) (layer "F.Cu") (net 6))
 (segment (start 32.9375 22) (end 53.225 10) (width 0.25) (layer "F.Cu") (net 6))
 (segment (start 53.225 10) (end 80 26.825) (width 0.35) (layer "F.Cu") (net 6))
 (segment (start 12.9375 22) (end 53.225 10) (width 0.25) (layer "F.Cu") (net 6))
 (segment (start 72.9375 22) (end 53.225 10) (width 0.25) (layer "F.Cu") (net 6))
 (segment (start 53.225 10) (end 27.175 28) (width 0.3) (layer "F.Cu") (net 6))
 (segment (start 53.225 10) (end 7.175 28) (width 0.3) (layer "F.Cu") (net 6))
 (via (at 53.225 10) (size 0.8) (drill 0.4) (layers "F.Cu" "B.Cu") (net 6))
 (segment (start 80 41.08) (end 83 41.08) (width 0.35) (layer "B.Cu") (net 6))
 (segment (start 53.225 4) (end 53.225 10) (width 0.35) (layer "B.Cu") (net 6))
 (segment (start 83 41.08) (end 83 4) (width 0.35) (layer "B.Cu") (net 6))
 (segment (start 83 4) (end 53.225 4) (width 0.35) (layer "B.Cu") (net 6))
 (segment (start 10 10) (end 19.8625 10) (width 0.6) (layer "F.Cu") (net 13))
 (segment (start 24.1375 10) (end 32 10) (width 0.6) (layer "F.Cu") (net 1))
 (segment (start 45.05 10) (end 45.05 2) (width 0.5) (layer "F.Cu") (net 1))
 (segment (start 32 10) (end 40 10) (width 0.6) (layer "F.Cu") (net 1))
 (segment (start 40 10) (end 45.05 10) (width 0.6) (layer "F.Cu") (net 1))
 (via (at 45.05 2) (size 0.8) (drill 0.4) (layers "F.Cu" "B.Cu") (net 1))
 (segment (start 32 58) (end 12 58) (width 0.5) (layer "B.Cu") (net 1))
 (segment (start 86 58) (end 72 58) (width 0.5) (layer "B.Cu") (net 1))
 (segment (start 86 2) (end 86 58) (width 0.5) (layer "B.Cu") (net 1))
 (segment (start 45.05 2) (end 86 2) (width 0.5) (layer "B.Cu") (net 1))
 (segment (start 72 58) (end 52 58) (width 0.5) (layer "B.Cu") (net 1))
 (segment (start 52 58) (end 32 58) (width 0.5) (layer "B.Cu") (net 1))
 (segment (start 80 25.175) (end 81.27 16.73) (width 0.25) (layer "F.Cu") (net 7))
 (segment (start 83 38.54) (end 83 25.175) (width 0.25) (layer "F.Cu") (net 7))
 (segment (start 45 34) (end 81.27 16.73) (width 0.25) (layer "F.Cu") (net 7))
 (segment (start 83 25.175) (end 80 25.175) (width 0.25) (layer "F.Cu") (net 7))
 (segment (start 80 38.54) (end 83 38.54) (width 0.25) (layer "F.Cu") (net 7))
 (segment (start 37.38 25.08) (end 7.175 34) (width 0.25) (layer "F.Cu") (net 22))
 (segment (start 37.38 27.62) (end 27.175 34) (width 0.25) (layer "F.Cu") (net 24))
 (segment (start 37.38 30.16) (end 47.175 34) (width 0.25) (layer "F.Cu") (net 17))
 (segment (start 37.38 32.7) (end 67.175 34) (width 0.25) (layer "F.Cu") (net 9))
 (segment (start 8.825 34) (end 11.0625 41.05) (width 0.25) (layer "F.Cu") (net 23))
 (segment (start 15.175 34) (end 11.0625 41.05) (width 0.25) (layer "F.Cu") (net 23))
 (segment (start 28.825 34) (end 31.0625 41.05) (width 0.25) (layer "F.Cu") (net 8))
 (segment (start 35.175 34) (end 31.0625 41.05) (width 0.25) (layer "F.Cu") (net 8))
 (segment (start 48.825 34) (end 51.0625 41.05) (width 0.25) (layer "F.Cu") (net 18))
 (segment (start 55.175 34) (end 51.0625 41.05) (width 0.25) (layer "F.Cu") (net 18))
 (segment (start 75.175 34) (end 71.0625 41.05) (width 0.25) (layer "F.Cu") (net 10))
 (segment (start 68.825 34) (end 71.0625 41.05) (width 0.25) (layer "F.Cu") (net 10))
 (segment (start 12.9375 42) (end 12 65.62) (width 0.3) (layer "F.Cu") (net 12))
 (segment (start 32.9375 42) (end 32 65.62) (width 0.3) (layer "F.Cu") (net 4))
 (segment (start 52.9375 42) (end 52 65.62) (width 0.3) (layer "F.Cu") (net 16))
 (segment (start 72.9375 42) (end 72 65.62) (width 0.3) (layer "F.Cu") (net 26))
 (segment (start 12 63.08) (end 15.175 28) (width 0.25) (layer "F.Cu") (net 11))
 (segment (start 32 63.08) (end 35.175 28) (width 0.25) (layer "F.Cu") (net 3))
 (segment (start 52 63.08) (end 55.175 28) (width 0.25) (layer "F.Cu") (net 14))
 (segment (start 72 63.08) (end 75.175 28) (width 0.25) (layer "F.Cu") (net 25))
 (segment (start 52.62 27.62) (end 8.825 28) (width 0.25) (layer "F.Cu") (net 20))
 (segment (start 16.825 28) (end 8.825 28) (width 0.25) (layer "F.Cu") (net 20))
 (segment (start 11.0625 21.05) (end 8.825 28) (width 0.25) (layer "F.Cu") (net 20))
 (segment (start 31.0625 21.05) (end 28.825 28) (width 0.25) (layer "F.Cu") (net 21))
 (segment (start 52.62 30.16) (end 28.825 28) (width 0.25) (layer "F.Cu") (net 21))
 (segment (start 36.825 28) (end 28.825 28) (width 0.25) (layer "F.Cu") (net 21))
 (segment (start 52.62 32.7) (end 48.825 28) (width 0.25) (layer "F.Cu") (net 15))
 (segment (start 51.0625 21.05) (end 48.825 28) (width 0.25) (layer "F.Cu") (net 15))
 (segment (start 56.825 28) (end 48.825 28) (width 0.25) (layer "F.Cu") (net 15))
 (segment (start 71.0625 21.05) (end 68.825 28) (width 0.25) (layer "F.Cu") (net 5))
 (segment (start 52.62 37.78) (end 68.825 28) (width 0.25) (layer "F.Cu") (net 5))
 (segment (start 76.825 28) (end 68.825 28) (width 0.25) (layer "F.Cu") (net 5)))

